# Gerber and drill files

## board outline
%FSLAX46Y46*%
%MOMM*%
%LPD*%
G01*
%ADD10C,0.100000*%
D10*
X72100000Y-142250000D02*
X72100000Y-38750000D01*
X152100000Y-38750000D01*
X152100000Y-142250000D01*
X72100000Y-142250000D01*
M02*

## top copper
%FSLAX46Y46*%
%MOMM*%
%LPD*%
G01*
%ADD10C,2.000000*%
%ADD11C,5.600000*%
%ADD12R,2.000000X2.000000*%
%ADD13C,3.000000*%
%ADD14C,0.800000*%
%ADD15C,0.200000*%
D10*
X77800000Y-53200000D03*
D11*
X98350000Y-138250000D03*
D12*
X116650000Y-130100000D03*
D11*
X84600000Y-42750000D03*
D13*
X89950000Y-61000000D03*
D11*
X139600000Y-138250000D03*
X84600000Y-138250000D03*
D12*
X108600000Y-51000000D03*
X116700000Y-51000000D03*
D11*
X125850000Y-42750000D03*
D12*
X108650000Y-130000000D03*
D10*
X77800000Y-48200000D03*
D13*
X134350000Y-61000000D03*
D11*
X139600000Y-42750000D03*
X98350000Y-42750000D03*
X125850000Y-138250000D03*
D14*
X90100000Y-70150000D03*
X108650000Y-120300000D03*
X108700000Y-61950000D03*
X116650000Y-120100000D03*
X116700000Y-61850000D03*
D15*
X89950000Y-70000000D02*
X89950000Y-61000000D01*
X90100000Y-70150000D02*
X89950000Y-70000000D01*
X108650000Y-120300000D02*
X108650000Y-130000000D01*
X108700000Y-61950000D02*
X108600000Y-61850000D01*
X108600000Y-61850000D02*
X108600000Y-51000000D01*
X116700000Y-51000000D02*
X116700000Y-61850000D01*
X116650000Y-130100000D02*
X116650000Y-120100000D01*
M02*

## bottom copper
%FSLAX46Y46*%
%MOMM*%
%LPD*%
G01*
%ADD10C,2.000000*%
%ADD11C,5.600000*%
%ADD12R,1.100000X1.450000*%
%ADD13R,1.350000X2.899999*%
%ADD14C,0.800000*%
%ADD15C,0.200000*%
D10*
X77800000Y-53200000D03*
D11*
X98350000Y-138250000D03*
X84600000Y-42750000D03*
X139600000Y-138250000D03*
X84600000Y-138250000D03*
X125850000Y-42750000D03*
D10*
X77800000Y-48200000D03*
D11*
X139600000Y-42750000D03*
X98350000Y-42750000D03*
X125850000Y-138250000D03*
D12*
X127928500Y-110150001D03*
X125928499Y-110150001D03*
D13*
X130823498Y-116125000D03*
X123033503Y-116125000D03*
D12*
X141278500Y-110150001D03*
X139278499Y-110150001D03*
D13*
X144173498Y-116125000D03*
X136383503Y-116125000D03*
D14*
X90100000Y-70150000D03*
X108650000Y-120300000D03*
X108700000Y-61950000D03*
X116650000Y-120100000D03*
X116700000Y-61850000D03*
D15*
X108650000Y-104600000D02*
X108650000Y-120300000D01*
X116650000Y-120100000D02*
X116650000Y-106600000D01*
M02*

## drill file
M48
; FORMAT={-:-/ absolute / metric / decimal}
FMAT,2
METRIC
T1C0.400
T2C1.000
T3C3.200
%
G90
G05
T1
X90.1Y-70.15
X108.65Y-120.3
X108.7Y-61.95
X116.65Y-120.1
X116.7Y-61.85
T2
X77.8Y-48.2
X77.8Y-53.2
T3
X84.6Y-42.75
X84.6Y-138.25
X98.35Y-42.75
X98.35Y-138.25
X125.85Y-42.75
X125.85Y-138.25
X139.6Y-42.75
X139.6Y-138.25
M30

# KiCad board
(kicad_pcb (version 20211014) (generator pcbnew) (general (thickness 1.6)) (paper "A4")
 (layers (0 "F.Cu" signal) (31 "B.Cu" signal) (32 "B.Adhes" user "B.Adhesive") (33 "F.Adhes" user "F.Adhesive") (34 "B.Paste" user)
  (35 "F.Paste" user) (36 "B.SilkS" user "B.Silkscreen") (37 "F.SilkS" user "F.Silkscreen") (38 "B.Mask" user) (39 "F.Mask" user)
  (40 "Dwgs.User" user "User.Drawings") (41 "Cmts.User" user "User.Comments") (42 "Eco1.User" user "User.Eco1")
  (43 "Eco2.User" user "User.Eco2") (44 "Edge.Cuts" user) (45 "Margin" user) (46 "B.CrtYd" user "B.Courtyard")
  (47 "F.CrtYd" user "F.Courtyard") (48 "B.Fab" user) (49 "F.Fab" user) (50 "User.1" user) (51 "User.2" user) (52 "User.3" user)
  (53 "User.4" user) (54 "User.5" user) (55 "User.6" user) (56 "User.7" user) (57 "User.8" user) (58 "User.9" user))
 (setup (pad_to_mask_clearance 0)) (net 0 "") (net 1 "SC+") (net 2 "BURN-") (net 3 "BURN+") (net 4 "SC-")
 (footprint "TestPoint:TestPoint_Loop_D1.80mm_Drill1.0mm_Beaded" (layer "F.Cu") (at 77.85 53.2)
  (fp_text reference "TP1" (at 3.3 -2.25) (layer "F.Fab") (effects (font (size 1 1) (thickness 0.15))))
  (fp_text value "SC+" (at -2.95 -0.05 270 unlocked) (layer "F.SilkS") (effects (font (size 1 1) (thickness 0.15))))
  (pad "1" thru_hole circle (at -0.05 0) (size 2 2) (drill 1) (layers *.Cu *.Mask) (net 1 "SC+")))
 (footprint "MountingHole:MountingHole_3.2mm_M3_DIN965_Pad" (layer "F.Cu") (at 98.35 138.25)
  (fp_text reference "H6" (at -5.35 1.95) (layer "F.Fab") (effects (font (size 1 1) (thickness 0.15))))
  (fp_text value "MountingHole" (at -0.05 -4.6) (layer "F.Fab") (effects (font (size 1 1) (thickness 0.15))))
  (pad "1" thru_hole circle (at 0 0) (size 5.6 5.6) (drill 3.2) (layers *.Cu *.Mask)))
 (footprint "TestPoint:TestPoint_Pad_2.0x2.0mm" (layer "F.Cu") (at 116.65 130.1)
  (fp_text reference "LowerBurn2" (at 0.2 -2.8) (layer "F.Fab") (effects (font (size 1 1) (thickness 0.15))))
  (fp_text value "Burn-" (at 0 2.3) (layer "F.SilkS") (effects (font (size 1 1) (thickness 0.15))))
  (pad "1" smd rect (at 0 0) (size 2 2) (layers "F.Cu" "F.Mask") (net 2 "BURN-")))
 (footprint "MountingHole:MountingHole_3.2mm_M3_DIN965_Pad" (layer "F.Cu") (at 84.6 42.75)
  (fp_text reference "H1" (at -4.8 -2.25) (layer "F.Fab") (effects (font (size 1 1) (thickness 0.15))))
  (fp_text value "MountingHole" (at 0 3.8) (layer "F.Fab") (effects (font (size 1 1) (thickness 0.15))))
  (pad "1" thru_hole circle (at 0 0) (size 5.6 5.6) (drill 3.2) (layers *.Cu *.Mask)))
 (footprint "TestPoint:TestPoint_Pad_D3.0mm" (layer "F.Cu") (at 89.95 61)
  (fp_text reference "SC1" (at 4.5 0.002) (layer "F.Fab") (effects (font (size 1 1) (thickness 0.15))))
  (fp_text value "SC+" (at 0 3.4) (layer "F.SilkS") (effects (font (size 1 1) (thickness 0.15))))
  (pad "1" smd circle (at 0 0) (size 3 3) (layers "F.Cu" "F.Mask") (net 1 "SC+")))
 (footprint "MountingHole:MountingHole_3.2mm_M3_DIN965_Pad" (layer "F.Cu") (at 139.6 138.25)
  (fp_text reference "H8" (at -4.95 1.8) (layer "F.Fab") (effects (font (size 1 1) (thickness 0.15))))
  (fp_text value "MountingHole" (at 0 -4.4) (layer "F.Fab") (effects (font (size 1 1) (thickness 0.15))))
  (pad "1" thru_hole circle (at 0 0) (size 5.6 5.6) (drill 3.2) (layers *.Cu *.Mask)))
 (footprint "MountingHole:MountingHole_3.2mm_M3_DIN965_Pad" (layer "F.Cu") (at 84.6 138.25)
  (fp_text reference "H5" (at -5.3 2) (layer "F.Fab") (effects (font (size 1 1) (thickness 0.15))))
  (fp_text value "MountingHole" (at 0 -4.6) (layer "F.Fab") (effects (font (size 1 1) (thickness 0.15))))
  (pad "1" thru_hole circle (at 0 0) (size 5.6 5.6) (drill 3.2) (layers *.Cu *.Mask)))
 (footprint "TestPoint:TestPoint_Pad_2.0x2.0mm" (layer "F.Cu") (at 108.6 51)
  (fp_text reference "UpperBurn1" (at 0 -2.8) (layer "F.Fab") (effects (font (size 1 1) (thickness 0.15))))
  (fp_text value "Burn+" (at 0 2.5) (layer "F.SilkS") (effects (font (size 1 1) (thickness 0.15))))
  (pad "1" smd rect (at 0 0) (size 2 2) (layers "F.Cu" "F.Mask") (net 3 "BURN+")))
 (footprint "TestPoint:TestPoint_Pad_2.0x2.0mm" (layer "F.Cu") (at 116.7 51)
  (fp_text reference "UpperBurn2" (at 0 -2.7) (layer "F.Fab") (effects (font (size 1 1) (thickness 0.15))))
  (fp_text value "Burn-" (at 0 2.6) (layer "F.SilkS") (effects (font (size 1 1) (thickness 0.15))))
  (pad "1" smd rect (at 0 0) (size 2 2) (layers "F.Cu" "F.Mask") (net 2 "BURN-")))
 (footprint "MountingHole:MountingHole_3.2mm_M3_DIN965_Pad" (layer "F.Cu") (at 125.85 42.75)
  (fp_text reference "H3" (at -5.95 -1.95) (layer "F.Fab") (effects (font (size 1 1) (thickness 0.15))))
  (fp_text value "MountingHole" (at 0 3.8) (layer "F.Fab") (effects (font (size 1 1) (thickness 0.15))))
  (pad "1" thru_hole circle (at 0 0) (size 5.6 5.6) (drill 3.2) (layers *.Cu *.Mask)))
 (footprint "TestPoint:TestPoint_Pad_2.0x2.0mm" (layer "F.Cu") (at 108.65 130)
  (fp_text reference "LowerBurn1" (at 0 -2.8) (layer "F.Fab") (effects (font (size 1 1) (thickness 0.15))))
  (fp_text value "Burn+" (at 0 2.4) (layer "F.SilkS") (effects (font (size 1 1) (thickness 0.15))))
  (pad "1" smd rect (at 0 0) (size 2 2) (layers "F.Cu" "F.Mask") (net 3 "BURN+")))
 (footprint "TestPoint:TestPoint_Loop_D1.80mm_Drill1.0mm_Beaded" (layer "F.Cu") (at 77.8 48.3)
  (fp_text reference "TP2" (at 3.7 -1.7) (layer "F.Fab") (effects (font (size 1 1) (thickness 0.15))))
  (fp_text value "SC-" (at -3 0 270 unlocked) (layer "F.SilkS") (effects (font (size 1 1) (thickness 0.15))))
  (pad "1" thru_hole circle (at 0 -0.1) (size 2 2) (drill 1) (layers *.Cu *.Mask) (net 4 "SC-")))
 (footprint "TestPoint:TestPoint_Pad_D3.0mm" (layer "F.Cu") (at 134.35 61)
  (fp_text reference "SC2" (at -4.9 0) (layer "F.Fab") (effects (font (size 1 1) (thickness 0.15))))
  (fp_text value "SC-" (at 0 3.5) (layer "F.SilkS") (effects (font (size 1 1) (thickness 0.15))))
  (pad "1" smd circle (at 0 0) (size 3 3) (layers "F.Cu" "F.Mask") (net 4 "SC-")))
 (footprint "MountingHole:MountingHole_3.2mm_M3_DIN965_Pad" (layer "F.Cu") (at 139.6 42.75)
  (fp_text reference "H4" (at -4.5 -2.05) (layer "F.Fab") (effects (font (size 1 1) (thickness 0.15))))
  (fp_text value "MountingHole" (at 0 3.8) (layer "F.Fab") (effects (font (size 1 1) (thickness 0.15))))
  (pad "1" thru_hole circle (at 0 0) (size 5.6 5.6) (drill 3.2) (layers *.Cu *.Mask)))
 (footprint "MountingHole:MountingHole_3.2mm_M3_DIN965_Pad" (layer "F.Cu") (at 98.35 42.75)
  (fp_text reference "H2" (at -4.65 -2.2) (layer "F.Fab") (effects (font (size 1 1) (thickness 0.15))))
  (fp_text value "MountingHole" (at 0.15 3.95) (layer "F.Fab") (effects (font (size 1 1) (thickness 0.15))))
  (pad "1" thru_hole circle (at 0 0) (size 5.6 5.6) (drill 3.2) (layers *.Cu *.Mask)))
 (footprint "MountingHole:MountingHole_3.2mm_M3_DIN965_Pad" (layer "F.Cu") (at 125.85 138.25)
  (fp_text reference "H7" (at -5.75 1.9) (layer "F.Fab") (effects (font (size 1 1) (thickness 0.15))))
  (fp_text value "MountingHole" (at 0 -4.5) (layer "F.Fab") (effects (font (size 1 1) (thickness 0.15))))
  (pad "1" thru_hole circle (at 0 0) (size 5.6 5.6) (drill 3.2) (layers *.Cu *.Mask)))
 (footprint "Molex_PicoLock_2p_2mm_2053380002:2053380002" (layer "B.Cu") (at 127.9285 110.150001)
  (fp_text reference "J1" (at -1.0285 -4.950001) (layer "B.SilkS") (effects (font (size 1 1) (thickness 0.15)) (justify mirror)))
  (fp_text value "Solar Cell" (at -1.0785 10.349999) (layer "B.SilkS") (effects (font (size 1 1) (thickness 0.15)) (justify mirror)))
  (pad "1" smd rect locked (at 0 0) (size 1.1 1.45) (layers "B.Cu" "B.Paste" "B.Mask") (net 4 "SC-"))
  (pad "2" smd rect locked (at -2.000001 0) (size 1.1 1.45) (layers "B.Cu" "B.Paste" "B.Mask") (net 1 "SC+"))
  (pad "3" smd rect locked (at 2.894998 5.974999) (size 1.35 2.899999) (layers "B.Cu" "B.Paste" "B.Mask"))
  (pad "4" smd rect locked (at -4.894997 5.974999) (size 1.35 2.899999) (layers "B.Cu" "B.Paste" "B.Mask")))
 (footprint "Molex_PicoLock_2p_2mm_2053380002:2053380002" (layer "B.Cu") (at 141.2785 110.150001)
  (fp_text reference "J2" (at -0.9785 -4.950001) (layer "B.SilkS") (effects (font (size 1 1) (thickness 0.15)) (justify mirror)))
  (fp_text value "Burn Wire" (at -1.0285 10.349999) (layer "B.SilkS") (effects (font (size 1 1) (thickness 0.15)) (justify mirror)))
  (pad "1" smd rect locked (at 0 0) (size 1.1 1.45) (layers "B.Cu" "B.Paste" "B.Mask") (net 2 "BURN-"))
  (pad "2" smd rect locked (at -2.000001 0) (size 1.1 1.45) (layers "B.Cu" "B.Paste" "B.Mask") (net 3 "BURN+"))
  (pad "3" smd rect locked (at 2.894998 5.974999) (size 1.35 2.899999) (layers "B.Cu" "B.Paste" "B.Mask"))
  (pad "4" smd rect locked (at -4.894997 5.974999) (size 1.35 2.899999) (layers "B.Cu" "B.Paste" "B.Mask")))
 (gr_poly (pts (xy 72.1 142.25) (xy 72.1 38.75) (xy 152.1 38.75) (xy 152.1 142.25)) (layer "Edge.Cuts") (width 0.1) (fill none))
 (segment (start 89.95 70) (end 89.95 61) (width 0.2) (layer "F.Cu") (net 1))
 (segment (start 90.1 70.15) (end 89.95 70) (width 0.2) (layer "F.Cu") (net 1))
 (via (at 90.1 70.15) (size 0.8) (drill 0.4) (layers "F.Cu" "B.Cu") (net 1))
 (segment (start 108.65 120.3) (end 108.65 130) (width 0.2) (layer "F.Cu") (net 3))
 (segment (start 108.7 61.95) (end 108.6 61.85) (width 0.2) (layer "F.Cu") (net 3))
 (segment (start 108.6 61.85) (end 108.6 51) (width 0.2) (layer "F.Cu") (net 3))
 (via (at 108.65 120.3) (size 0.8) (drill 0.4) (layers "F.Cu" "B.Cu") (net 3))
 (via (at 108.7 61.95) (size 0.8) (drill 0.4) (layers "F.Cu" "B.Cu") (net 3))
 (segment (start 108.65 104.6) (end 108.65 120.3) (width 0.2) (layer "B.Cu") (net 3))
 (segment (start 116.7 51) (end 116.7 61.85) (width 0.2) (layer "F.Cu") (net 2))
 (segment (start 116.65 130.1) (end 116.65 120.1) (width 0.2) (layer "F.Cu") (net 2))
 (via (at 116.65 120.1) (size 0.8) (drill 0.4) (layers "F.Cu" "B.Cu") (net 2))
 (via (at 116.7 61.85) (size 0.8) (drill 0.4) (layers "F.Cu" "B.Cu") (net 2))
 (segment (start 116.65 120.1) (end 116.65 106.6) (width 0.2) (layer "B.Cu") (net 2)))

